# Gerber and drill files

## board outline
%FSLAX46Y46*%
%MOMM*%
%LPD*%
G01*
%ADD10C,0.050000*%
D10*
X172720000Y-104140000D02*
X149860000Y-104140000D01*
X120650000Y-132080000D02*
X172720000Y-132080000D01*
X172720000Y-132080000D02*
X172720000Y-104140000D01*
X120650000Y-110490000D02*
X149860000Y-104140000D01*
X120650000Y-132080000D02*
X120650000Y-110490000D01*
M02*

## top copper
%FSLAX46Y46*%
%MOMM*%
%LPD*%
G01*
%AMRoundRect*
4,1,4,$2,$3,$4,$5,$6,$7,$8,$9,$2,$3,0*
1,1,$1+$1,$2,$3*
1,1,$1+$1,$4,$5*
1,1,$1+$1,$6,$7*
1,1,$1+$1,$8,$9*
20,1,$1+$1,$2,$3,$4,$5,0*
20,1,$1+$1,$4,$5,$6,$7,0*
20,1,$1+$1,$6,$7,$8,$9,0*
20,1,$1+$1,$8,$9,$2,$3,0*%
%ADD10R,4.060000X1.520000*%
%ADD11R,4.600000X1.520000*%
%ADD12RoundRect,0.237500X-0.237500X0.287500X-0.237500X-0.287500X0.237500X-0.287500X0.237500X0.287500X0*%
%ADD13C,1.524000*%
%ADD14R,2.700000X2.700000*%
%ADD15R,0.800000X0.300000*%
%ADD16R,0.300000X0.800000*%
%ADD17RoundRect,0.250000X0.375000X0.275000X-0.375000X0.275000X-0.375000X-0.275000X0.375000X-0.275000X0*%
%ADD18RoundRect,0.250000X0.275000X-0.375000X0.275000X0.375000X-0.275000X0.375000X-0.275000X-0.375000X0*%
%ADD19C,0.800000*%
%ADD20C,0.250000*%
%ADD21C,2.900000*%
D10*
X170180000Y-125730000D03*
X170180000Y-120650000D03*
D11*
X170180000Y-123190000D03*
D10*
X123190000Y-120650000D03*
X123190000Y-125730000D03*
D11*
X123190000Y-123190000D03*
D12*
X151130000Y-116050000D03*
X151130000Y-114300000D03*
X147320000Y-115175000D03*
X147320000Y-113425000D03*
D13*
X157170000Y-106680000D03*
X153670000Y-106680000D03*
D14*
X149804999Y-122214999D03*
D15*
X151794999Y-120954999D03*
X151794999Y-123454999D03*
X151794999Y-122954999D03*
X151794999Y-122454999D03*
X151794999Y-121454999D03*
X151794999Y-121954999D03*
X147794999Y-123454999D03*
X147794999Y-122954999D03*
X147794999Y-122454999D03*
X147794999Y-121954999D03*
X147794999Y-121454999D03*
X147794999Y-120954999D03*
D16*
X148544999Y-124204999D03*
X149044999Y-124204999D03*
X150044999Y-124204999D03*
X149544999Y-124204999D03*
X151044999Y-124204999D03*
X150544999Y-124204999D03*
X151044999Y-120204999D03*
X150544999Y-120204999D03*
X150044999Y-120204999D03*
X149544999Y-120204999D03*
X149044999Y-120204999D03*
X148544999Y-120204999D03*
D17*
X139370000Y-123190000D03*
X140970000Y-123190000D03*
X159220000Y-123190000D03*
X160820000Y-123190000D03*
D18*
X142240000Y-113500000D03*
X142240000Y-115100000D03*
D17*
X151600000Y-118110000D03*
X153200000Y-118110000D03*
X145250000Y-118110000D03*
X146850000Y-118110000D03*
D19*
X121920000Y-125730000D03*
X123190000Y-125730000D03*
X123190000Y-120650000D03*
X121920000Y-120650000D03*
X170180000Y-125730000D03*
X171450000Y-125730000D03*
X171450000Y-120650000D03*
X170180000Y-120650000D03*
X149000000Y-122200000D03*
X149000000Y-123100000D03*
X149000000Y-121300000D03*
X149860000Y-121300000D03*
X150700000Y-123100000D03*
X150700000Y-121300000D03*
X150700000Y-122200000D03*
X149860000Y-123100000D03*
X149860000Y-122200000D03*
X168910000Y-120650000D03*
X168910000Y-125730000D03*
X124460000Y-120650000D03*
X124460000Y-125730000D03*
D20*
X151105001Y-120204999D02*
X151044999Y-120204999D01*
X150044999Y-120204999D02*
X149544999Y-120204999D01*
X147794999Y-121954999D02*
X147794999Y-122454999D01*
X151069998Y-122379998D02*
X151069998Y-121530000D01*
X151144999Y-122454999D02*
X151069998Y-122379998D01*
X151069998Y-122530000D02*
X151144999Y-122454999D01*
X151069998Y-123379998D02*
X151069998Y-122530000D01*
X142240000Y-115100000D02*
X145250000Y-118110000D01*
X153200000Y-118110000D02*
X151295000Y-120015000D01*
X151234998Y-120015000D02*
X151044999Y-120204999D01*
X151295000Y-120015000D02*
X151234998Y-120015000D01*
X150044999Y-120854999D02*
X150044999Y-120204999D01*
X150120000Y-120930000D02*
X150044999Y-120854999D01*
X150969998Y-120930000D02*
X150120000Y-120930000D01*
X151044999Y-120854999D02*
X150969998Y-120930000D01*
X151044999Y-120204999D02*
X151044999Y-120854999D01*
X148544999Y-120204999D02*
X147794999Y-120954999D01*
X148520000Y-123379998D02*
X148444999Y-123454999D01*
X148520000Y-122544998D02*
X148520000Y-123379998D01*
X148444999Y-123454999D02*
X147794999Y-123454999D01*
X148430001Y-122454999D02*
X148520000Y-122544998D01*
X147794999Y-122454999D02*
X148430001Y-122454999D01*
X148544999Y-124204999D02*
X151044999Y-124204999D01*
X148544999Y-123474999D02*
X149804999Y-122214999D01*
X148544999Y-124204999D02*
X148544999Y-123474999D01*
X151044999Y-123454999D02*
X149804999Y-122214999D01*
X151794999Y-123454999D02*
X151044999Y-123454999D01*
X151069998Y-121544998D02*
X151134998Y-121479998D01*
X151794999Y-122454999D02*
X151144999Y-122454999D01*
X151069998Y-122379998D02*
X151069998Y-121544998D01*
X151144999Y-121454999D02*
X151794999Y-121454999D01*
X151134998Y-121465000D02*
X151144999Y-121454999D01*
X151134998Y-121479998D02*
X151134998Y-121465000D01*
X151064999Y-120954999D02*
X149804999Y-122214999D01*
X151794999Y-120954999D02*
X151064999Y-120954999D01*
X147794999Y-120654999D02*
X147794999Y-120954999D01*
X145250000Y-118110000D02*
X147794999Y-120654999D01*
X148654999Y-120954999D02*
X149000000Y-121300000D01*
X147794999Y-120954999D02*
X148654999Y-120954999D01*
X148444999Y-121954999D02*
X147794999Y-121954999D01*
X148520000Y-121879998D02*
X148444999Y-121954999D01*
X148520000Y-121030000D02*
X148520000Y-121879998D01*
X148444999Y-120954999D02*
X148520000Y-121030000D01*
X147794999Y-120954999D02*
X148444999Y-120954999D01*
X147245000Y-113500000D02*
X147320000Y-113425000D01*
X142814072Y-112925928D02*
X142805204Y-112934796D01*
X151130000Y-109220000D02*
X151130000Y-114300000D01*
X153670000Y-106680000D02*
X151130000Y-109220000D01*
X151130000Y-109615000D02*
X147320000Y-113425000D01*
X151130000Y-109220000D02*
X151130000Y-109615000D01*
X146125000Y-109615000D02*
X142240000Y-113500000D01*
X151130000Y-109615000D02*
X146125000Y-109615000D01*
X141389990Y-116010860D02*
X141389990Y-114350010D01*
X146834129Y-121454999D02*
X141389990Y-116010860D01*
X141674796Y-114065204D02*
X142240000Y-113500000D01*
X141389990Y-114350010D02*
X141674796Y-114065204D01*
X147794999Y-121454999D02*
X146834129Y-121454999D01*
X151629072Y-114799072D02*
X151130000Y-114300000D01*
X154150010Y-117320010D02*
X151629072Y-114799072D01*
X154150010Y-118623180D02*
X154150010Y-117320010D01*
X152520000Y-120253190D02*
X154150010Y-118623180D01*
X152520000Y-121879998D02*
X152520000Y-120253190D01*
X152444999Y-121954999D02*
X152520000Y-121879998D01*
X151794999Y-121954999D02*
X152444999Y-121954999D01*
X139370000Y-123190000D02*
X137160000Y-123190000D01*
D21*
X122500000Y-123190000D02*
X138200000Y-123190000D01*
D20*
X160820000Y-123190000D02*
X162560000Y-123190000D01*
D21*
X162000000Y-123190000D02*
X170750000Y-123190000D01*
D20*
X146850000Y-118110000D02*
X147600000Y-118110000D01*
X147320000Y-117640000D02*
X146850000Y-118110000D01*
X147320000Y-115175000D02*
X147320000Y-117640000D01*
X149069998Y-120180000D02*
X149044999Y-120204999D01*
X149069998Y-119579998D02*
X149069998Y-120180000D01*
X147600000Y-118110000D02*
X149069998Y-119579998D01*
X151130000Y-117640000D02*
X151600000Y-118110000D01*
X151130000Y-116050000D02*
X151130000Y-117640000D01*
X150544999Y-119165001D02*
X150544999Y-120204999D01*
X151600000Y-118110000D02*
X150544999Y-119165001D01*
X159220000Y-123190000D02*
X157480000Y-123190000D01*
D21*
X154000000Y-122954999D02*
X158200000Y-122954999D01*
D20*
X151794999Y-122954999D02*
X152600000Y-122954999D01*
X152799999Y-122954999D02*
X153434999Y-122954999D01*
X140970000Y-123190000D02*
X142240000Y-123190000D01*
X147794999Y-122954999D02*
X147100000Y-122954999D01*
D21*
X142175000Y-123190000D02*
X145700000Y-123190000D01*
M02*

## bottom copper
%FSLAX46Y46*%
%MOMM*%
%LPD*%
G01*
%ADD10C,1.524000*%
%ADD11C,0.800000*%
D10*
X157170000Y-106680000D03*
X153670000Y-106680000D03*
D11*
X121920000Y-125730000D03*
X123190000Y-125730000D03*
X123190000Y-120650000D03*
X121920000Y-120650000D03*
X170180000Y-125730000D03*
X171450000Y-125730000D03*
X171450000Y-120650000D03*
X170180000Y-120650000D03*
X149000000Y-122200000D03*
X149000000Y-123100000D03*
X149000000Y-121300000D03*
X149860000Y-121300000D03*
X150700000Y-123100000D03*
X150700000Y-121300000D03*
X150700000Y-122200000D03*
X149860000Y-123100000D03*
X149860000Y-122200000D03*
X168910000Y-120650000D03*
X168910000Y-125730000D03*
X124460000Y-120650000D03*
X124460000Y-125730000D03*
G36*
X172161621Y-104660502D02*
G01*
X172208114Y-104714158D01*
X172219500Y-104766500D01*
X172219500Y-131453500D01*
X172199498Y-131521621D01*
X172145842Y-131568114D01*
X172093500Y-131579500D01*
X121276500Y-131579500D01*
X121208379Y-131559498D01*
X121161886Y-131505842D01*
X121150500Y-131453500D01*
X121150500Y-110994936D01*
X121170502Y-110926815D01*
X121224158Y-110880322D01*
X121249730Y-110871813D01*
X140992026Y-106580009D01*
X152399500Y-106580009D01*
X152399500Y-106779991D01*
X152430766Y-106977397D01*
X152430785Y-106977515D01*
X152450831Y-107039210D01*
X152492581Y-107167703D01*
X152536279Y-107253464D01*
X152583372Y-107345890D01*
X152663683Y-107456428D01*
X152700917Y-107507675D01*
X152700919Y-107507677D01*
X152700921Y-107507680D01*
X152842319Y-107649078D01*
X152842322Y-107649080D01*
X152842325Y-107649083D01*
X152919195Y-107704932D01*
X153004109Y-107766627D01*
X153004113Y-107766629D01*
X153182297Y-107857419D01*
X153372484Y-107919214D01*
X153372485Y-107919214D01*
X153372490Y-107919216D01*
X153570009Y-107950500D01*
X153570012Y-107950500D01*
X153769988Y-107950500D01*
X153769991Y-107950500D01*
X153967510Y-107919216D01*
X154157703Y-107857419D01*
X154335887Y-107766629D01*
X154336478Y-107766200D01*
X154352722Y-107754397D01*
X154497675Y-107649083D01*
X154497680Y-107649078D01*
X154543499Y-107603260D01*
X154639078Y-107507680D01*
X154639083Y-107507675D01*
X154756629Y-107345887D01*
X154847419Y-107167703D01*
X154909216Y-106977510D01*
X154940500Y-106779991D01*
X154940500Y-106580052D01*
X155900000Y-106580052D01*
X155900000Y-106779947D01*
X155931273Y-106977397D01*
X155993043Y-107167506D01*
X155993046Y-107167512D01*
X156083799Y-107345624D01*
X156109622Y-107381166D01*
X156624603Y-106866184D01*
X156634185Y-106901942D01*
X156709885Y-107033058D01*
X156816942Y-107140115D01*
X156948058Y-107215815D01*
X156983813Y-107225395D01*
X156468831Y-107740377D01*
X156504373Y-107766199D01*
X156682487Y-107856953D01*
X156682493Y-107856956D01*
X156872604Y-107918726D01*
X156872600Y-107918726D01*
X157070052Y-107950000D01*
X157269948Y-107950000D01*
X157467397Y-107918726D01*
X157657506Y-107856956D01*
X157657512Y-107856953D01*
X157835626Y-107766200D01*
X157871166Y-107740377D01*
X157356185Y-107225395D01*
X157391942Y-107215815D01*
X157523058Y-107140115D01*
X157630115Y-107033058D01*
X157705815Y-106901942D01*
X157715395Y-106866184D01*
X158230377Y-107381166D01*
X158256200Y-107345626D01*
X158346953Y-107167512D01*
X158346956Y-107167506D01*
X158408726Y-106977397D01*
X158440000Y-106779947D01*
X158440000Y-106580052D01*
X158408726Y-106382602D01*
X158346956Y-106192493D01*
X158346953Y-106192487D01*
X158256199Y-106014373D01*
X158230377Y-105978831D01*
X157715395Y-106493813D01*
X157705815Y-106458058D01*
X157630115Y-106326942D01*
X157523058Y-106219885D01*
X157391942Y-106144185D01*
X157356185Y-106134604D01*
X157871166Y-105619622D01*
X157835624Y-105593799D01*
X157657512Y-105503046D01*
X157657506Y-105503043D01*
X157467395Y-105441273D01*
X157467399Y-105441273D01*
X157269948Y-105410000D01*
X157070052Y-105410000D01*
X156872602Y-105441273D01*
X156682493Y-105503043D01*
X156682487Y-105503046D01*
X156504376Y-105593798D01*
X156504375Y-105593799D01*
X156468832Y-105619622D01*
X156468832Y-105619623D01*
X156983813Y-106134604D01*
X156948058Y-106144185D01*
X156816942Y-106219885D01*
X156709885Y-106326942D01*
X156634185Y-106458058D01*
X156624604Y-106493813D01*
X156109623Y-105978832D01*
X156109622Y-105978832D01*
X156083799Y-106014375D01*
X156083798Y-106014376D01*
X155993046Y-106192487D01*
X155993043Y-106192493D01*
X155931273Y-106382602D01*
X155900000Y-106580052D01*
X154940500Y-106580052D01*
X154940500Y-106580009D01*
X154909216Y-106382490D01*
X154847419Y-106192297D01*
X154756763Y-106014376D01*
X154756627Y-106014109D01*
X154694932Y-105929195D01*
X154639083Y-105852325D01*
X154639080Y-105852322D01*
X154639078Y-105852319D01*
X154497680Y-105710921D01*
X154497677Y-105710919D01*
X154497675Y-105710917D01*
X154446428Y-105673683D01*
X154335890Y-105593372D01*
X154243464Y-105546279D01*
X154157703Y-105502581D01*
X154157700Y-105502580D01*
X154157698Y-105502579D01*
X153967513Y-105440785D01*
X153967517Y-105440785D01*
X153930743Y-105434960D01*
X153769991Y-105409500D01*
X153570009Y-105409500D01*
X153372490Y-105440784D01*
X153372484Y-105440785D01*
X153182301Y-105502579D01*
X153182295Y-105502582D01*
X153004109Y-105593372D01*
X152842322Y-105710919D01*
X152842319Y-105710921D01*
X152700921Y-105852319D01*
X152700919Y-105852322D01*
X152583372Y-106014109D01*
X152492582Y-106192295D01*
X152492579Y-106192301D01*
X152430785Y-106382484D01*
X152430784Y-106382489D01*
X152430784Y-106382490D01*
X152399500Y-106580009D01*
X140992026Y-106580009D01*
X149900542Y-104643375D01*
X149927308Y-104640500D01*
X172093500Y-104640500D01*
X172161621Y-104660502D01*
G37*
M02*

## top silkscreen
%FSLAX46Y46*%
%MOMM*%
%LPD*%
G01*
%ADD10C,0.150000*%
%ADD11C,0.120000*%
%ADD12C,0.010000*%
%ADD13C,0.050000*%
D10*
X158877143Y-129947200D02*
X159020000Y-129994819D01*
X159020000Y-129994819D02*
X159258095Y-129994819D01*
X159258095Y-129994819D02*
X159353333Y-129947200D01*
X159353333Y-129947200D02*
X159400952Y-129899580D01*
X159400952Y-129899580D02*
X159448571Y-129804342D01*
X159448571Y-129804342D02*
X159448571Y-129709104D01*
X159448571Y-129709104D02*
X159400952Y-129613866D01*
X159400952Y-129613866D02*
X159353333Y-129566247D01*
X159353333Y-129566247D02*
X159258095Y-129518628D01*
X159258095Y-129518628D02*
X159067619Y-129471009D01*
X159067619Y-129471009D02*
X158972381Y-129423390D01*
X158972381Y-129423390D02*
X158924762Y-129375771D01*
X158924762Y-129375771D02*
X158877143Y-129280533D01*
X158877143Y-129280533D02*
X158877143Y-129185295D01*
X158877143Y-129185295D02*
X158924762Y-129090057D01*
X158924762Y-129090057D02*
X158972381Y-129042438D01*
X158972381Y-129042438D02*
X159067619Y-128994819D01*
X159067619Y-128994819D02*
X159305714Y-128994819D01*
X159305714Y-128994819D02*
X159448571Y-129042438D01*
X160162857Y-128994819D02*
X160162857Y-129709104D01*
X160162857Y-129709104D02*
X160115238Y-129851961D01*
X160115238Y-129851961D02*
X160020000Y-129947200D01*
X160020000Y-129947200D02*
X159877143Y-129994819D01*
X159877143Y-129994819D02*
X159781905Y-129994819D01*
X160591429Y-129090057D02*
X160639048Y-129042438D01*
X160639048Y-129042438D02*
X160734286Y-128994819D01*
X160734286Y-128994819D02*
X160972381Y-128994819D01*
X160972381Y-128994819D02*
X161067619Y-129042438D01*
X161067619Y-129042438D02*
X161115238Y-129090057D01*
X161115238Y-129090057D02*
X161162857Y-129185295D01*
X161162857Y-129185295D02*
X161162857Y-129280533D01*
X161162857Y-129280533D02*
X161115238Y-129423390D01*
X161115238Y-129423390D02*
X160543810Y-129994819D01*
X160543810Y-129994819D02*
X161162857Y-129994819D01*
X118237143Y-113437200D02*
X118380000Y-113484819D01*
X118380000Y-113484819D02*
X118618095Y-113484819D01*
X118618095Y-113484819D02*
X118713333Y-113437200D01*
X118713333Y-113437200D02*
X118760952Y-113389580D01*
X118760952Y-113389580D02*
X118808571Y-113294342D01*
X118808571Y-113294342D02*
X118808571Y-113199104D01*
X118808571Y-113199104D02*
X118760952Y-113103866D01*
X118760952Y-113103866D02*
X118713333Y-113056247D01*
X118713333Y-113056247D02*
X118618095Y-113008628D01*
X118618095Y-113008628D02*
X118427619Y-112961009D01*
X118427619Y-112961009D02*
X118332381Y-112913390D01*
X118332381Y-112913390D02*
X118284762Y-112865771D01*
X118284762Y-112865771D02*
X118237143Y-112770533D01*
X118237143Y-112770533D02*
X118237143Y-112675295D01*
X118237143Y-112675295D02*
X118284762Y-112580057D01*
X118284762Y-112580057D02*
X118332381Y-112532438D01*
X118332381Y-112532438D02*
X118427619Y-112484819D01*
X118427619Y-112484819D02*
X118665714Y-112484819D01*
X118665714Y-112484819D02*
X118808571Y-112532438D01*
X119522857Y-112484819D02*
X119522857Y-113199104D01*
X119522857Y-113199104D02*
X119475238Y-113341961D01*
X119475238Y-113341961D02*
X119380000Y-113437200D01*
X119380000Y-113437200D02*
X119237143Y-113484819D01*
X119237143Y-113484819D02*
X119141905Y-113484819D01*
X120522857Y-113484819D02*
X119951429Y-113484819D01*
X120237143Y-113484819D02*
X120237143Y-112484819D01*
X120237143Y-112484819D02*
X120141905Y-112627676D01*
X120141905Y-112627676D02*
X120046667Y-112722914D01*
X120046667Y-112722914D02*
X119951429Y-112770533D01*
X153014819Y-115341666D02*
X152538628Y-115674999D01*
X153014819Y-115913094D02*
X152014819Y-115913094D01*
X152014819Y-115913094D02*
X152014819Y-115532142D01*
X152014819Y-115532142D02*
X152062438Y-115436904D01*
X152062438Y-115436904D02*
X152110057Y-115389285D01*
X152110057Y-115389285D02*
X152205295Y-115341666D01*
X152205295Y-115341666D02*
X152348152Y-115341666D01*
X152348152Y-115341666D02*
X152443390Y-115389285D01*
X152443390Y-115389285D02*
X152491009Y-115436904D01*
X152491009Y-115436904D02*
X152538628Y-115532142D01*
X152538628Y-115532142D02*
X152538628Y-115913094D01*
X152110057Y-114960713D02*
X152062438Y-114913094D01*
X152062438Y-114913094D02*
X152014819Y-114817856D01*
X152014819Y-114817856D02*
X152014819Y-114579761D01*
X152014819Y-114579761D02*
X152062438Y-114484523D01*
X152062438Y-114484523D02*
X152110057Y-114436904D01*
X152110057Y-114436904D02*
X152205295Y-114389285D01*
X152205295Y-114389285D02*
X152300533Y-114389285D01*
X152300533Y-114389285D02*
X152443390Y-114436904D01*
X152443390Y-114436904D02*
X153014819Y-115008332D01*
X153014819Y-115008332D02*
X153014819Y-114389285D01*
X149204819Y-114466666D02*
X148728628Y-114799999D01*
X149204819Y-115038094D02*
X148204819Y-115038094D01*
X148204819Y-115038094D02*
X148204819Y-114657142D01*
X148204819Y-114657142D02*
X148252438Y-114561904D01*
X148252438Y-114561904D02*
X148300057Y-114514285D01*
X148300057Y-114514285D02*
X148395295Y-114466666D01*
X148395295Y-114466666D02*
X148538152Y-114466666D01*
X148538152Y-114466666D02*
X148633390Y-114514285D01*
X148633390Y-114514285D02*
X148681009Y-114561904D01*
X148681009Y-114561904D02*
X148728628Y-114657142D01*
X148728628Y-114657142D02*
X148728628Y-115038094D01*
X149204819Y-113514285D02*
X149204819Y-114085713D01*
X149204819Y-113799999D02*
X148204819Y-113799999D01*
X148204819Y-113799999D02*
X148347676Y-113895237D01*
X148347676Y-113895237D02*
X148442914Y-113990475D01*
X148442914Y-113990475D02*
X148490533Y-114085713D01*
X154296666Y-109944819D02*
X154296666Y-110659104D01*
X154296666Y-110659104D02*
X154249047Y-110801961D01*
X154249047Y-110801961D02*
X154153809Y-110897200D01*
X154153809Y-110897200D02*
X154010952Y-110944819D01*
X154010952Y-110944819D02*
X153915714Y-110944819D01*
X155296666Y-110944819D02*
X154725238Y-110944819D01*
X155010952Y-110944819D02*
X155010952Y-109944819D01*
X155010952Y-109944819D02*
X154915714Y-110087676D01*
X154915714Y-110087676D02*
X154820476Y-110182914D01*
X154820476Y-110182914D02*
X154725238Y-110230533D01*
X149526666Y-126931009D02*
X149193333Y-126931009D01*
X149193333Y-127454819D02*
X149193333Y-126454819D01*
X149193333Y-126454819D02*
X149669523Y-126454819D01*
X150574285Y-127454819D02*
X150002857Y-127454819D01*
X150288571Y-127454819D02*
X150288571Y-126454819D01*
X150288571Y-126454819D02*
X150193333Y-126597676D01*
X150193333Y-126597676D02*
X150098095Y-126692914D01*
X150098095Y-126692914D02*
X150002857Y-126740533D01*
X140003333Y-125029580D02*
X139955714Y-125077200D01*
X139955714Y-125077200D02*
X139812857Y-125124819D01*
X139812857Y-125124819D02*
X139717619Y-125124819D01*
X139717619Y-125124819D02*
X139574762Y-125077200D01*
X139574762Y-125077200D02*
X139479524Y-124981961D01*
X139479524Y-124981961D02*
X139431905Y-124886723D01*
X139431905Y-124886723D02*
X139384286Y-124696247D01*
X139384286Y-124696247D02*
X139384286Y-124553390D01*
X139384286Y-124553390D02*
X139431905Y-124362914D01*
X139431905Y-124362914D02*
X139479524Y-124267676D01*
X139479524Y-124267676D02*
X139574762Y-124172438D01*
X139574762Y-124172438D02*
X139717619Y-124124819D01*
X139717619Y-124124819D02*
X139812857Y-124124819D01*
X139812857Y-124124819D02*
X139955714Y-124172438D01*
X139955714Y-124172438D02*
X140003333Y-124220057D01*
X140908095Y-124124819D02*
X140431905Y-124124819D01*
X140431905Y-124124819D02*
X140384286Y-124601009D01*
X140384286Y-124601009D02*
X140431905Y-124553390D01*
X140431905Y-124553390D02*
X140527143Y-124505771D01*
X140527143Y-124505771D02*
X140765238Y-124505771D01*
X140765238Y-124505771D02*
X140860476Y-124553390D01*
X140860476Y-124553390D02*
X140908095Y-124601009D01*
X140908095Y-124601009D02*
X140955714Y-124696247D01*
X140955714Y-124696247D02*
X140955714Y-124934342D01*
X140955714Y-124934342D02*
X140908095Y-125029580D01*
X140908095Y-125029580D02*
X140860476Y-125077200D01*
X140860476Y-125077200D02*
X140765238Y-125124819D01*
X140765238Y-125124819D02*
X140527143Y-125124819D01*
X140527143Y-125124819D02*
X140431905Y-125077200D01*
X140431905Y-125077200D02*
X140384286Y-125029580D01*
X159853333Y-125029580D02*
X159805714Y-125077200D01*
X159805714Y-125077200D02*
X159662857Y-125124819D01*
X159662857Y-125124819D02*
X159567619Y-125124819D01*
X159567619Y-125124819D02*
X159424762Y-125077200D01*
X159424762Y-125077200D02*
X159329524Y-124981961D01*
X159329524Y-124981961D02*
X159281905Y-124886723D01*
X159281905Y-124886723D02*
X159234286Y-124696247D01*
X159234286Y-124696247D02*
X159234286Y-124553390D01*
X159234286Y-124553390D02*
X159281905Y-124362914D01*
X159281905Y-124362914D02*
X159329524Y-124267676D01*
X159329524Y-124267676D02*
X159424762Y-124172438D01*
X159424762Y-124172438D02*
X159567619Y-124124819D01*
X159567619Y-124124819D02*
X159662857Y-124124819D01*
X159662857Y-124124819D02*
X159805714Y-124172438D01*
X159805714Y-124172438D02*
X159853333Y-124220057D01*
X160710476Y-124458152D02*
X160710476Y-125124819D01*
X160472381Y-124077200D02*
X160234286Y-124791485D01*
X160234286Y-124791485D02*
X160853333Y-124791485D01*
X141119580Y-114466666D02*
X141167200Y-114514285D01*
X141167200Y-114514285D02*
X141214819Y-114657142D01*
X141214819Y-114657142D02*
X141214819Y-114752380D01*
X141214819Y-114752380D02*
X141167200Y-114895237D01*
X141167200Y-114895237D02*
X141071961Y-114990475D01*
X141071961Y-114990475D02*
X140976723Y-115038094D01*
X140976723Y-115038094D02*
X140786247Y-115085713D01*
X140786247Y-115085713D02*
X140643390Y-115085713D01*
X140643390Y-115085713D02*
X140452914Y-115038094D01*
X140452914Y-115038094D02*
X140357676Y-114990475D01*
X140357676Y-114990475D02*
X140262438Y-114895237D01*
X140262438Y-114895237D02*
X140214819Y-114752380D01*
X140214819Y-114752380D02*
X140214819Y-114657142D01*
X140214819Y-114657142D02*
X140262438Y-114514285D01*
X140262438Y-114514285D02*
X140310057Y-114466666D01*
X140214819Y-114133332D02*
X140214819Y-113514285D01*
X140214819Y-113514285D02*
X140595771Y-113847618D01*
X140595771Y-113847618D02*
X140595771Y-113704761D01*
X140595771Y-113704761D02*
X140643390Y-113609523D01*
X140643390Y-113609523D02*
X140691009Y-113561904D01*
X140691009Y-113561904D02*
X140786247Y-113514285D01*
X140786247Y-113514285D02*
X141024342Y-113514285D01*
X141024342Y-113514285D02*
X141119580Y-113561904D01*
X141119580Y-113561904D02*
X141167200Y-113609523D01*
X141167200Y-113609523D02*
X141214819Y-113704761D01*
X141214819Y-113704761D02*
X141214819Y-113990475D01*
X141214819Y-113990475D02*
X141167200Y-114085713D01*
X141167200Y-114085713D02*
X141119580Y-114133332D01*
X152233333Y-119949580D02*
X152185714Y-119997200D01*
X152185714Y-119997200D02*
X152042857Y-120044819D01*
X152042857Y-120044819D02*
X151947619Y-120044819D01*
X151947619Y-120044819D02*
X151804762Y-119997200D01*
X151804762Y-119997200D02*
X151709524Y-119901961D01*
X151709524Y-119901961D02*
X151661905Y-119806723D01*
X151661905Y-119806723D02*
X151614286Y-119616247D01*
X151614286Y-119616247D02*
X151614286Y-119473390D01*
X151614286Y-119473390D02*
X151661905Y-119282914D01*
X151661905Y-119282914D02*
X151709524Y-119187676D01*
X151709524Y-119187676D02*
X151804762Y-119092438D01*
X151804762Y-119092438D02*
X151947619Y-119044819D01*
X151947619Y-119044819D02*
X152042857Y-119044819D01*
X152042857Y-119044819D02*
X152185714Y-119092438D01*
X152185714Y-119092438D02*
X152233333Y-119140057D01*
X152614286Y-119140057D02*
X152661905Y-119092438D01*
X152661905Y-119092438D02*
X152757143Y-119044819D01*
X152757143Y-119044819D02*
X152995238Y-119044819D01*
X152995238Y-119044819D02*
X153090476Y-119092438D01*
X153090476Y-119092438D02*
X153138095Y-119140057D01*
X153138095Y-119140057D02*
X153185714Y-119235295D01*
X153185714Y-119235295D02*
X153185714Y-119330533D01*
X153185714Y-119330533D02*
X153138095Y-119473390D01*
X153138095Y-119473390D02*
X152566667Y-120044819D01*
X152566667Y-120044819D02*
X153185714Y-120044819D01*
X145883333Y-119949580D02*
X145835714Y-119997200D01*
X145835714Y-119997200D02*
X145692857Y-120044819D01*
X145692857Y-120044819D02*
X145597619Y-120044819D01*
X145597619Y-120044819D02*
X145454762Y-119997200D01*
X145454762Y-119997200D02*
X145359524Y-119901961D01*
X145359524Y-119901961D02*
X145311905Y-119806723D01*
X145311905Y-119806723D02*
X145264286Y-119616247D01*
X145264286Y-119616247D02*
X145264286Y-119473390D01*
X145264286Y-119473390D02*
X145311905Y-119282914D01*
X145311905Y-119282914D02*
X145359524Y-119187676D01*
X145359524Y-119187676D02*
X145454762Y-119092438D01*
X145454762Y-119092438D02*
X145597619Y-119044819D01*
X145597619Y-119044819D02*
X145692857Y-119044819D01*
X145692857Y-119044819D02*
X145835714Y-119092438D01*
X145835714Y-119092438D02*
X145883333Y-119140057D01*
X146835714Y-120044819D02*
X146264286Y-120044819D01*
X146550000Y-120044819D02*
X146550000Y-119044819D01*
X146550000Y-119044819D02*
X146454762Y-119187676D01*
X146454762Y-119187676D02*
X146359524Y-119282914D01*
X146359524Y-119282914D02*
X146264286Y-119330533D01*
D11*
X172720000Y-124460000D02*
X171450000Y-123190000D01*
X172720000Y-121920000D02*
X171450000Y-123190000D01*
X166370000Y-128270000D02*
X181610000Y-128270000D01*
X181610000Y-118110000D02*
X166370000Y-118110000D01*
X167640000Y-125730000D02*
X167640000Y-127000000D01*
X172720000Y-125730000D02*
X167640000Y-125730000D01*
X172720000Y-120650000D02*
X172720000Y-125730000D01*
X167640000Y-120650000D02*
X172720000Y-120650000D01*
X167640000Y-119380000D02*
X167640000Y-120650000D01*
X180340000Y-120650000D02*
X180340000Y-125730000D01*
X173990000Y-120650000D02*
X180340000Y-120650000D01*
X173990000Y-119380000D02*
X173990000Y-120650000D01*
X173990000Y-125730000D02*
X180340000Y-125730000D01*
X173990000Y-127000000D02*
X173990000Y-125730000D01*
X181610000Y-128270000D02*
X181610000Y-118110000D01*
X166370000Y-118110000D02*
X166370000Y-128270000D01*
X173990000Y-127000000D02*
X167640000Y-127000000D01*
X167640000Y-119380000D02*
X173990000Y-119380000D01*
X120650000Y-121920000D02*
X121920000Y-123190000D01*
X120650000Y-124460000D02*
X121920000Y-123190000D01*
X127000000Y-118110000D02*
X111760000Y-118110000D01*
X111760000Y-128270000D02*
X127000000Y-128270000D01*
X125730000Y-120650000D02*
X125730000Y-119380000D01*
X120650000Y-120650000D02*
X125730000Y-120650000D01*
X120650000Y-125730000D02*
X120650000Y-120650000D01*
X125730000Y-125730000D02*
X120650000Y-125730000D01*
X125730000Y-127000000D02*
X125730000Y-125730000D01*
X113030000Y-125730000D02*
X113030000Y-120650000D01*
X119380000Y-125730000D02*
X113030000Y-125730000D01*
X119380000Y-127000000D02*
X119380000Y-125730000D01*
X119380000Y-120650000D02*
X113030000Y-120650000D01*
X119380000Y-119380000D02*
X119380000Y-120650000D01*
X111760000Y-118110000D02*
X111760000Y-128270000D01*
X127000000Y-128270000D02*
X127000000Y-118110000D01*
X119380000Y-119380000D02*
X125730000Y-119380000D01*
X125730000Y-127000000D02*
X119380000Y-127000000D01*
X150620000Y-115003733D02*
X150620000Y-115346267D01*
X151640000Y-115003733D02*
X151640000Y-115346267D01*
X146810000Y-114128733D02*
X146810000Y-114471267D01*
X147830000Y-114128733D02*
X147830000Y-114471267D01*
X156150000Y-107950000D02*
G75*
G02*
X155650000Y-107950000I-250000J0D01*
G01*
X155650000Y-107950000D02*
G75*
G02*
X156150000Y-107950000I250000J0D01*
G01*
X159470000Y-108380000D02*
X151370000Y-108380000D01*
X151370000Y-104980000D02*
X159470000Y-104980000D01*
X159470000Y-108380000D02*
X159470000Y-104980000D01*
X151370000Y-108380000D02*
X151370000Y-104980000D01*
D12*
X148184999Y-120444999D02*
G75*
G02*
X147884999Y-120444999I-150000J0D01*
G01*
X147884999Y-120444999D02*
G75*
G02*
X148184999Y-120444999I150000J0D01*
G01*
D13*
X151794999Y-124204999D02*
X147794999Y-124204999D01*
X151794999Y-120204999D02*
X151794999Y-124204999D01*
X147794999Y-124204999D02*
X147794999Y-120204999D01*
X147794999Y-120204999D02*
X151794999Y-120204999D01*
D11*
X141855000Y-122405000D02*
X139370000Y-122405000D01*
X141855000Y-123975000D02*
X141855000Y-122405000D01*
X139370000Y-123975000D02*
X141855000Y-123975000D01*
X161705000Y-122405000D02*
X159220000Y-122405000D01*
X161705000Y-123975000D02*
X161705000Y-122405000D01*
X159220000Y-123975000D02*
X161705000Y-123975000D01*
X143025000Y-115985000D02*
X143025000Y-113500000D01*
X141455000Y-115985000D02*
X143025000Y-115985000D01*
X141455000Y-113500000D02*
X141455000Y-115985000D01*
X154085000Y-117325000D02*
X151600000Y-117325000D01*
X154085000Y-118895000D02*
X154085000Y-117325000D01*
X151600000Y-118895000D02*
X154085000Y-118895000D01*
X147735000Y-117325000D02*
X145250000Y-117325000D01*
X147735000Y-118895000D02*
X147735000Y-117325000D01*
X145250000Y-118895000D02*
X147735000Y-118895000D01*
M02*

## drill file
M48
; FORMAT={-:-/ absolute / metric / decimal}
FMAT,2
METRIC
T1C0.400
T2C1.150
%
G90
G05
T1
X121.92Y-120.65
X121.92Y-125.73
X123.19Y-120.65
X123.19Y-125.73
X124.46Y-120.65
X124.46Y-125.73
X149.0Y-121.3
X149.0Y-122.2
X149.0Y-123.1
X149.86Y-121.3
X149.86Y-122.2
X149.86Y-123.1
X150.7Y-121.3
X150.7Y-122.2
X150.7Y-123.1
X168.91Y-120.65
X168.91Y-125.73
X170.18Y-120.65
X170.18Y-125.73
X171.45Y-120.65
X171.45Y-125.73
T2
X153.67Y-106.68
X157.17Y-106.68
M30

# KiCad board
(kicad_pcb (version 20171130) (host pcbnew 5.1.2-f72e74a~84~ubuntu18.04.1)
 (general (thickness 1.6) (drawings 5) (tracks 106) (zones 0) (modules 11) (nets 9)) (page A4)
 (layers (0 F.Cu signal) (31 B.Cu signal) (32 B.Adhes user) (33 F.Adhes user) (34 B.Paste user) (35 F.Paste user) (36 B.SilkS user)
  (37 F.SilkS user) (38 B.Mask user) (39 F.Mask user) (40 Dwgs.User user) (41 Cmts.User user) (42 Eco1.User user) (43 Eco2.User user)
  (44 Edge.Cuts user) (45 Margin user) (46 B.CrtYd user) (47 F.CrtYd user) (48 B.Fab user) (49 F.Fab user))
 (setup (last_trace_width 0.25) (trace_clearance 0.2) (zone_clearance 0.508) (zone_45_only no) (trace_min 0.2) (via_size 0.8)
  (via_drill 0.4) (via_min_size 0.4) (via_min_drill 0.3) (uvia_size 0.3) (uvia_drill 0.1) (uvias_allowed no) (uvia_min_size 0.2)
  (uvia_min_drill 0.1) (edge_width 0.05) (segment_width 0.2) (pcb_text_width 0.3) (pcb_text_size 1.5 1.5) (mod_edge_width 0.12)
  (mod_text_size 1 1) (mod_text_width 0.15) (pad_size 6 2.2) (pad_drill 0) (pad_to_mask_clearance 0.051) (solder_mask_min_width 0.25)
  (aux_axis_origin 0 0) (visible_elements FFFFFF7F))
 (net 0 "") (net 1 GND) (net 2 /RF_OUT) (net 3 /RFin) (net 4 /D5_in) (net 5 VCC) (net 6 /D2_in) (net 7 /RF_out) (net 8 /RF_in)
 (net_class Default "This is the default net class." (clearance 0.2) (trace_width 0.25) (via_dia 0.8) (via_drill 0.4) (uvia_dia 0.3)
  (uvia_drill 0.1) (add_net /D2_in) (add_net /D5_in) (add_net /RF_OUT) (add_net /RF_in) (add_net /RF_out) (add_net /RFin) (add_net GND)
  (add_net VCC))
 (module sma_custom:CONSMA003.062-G (layer F.Cu) (at 173.99 125.73)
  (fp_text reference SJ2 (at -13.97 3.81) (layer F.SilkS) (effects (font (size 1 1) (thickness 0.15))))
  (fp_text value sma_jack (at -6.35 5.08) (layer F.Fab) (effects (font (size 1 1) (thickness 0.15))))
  (fp_line (start -1.27 -1.27) (end -2.54 -2.54) (layer F.SilkS) (width 0.12))
  (fp_line (start -1.27 -3.81) (end -2.54 -2.54) (layer F.SilkS) (width 0.12))
  (fp_line (start -7.62 2.54) (end 7.62 2.54) (layer F.SilkS) (width 0.12))
  (fp_line (start 7.62 -7.62) (end -7.62 -7.62) (layer F.SilkS) (width 0.12))
  (fp_line (start -6.35 0) (end -6.35 1.27) (layer F.SilkS) (width 0.12))
  (fp_line (start -1.27 0) (end -6.35 0) (layer F.SilkS) (width 0.12))
  (fp_line (start -1.27 -5.08) (end -1.27 0) (layer F.SilkS) (width 0.12))
  (fp_line (start -6.35 -5.08) (end -1.27 -5.08) (layer F.SilkS) (width 0.12))
  (fp_line (start -6.35 -6.35) (end -6.35 -5.08) (layer F.SilkS) (width 0.12))
  (fp_line (start 6.35 -5.08) (end 6.35 0) (layer F.SilkS) (width 0.12))
  (fp_line (start 0 -5.08) (end 6.35 -5.08) (layer F.SilkS) (width 0.12))
  (fp_line (start 0 -6.35) (end 0 -5.08) (layer F.SilkS) (width 0.12))
  (fp_line (start 0 0) (end 6.35 0) (layer F.SilkS) (width 0.12))
  (fp_line (start 0 1.27) (end 0 0) (layer F.SilkS) (width 0.12))
  (fp_line (start 7.62 2.54) (end 7.62 -7.62) (layer F.SilkS) (width 0.12))
  (fp_line (start -7.62 -7.62) (end -7.62 2.54) (layer F.SilkS) (width 0.12))
  (fp_line (start 0 1.27) (end -6.35 1.27) (layer F.SilkS) (width 0.12))
  (fp_line (start -6.35 -6.35) (end 0 -6.35) (layer F.SilkS) (width 0.12))
  (pad 3 smd rect (at -3.81 0) (size 4.06 1.52) (layers F.Cu F.Paste F.Mask) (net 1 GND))
  (pad 2 smd rect (at -3.81 -5.08) (size 4.06 1.52) (layers F.Cu F.Paste F.Mask) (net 1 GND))
  (pad 1 smd rect (at -3.81 -2.54) (size 4.6 1.52) (layers F.Cu F.Paste F.Mask) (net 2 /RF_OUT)))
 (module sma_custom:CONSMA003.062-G (layer F.Cu) (at 119.38 120.65 180)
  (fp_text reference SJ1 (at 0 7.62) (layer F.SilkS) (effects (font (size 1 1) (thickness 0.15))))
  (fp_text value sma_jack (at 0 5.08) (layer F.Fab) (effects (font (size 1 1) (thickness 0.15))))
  (fp_line (start -1.27 -1.27) (end -2.54 -2.54) (layer F.SilkS) (width 0.12))
  (fp_line (start -1.27 -3.81) (end -2.54 -2.54) (layer F.SilkS) (width 0.12))
  (fp_line (start -7.62 2.54) (end 7.62 2.54) (layer F.SilkS) (width 0.12))
  (fp_line (start 7.62 -7.62) (end -7.62 -7.62) (layer F.SilkS) (width 0.12))
  (fp_line (start -6.35 0) (end -6.35 1.27) (layer F.SilkS) (width 0.12))
  (fp_line (start -1.27 0) (end -6.35 0) (layer F.SilkS) (width 0.12))
  (fp_line (start -1.27 -5.08) (end -1.27 0) (layer F.SilkS) (width 0.12))
  (fp_line (start -6.35 -5.08) (end -1.27 -5.08) (layer F.SilkS) (width 0.12))
  (fp_line (start -6.35 -6.35) (end -6.35 -5.08) (layer F.SilkS) (width 0.12))
  (fp_line (start 6.35 -5.08) (end 6.35 0) (layer F.SilkS) (width 0.12))
  (fp_line (start 0 -5.08) (end 6.35 -5.08) (layer F.SilkS) (width 0.12))
  (fp_line (start 0 -6.35) (end 0 -5.08) (layer F.SilkS) (width 0.12))
  (fp_line (start 0 0) (end 6.35 0) (layer F.SilkS) (width 0.12))
  (fp_line (start 0 1.27) (end 0 0) (layer F.SilkS) (width 0.12))
  (fp_line (start 7.62 2.54) (end 7.62 -7.62) (layer F.SilkS) (width 0.12))
  (fp_line (start -7.62 -7.62) (end -7.62 2.54) (layer F.SilkS) (width 0.12))
  (fp_line (start 0 1.27) (end -6.35 1.27) (layer F.SilkS) (width 0.12))
  (fp_line (start -6.35 -6.35) (end 0 -6.35) (layer F.SilkS) (width 0.12))
  (pad 3 smd rect (at -3.81 0 180) (size 4.06 1.52) (layers F.Cu F.Paste F.Mask) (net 1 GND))
  (pad 2 smd rect (at -3.81 -5.08 180) (size 4.06 1.52) (layers F.Cu F.Paste F.Mask) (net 1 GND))
  (pad 1 smd rect (at -3.81 -2.54 180) (size 4.6 1.52) (layers F.Cu F.Paste F.Mask) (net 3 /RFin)))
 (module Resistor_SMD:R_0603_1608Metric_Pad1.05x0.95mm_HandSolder (layer F.Cu) (at 151.13 115.175 270)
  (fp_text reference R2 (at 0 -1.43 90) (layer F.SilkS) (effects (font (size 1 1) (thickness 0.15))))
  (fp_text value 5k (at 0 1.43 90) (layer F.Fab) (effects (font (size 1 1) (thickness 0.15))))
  (fp_line (start -0.171267 0.51) (end 0.171267 0.51) (layer F.SilkS) (width 0.12))
  (fp_line (start -0.171267 -0.51) (end 0.171267 -0.51) (layer F.SilkS) (width 0.12))
  (pad 2 smd roundrect (at 0.875 0 270) (size 1.05 0.95) (layers F.Cu F.Paste F.Mask) (roundrect_rratio 0.25) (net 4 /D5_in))
  (pad 1 smd roundrect (at -0.875 0 270) (size 1.05 0.95) (layers F.Cu F.Paste F.Mask) (roundrect_rratio 0.25) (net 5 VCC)))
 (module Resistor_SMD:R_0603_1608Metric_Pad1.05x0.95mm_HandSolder (layer F.Cu) (at 147.32 114.3 270)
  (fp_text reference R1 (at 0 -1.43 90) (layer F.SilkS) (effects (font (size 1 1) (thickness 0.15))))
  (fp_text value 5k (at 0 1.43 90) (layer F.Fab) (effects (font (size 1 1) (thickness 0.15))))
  (fp_line (start -0.171267 0.51) (end 0.171267 0.51) (layer F.SilkS) (width 0.12))
  (fp_line (start -0.171267 -0.51) (end 0.171267 -0.51) (layer F.SilkS) (width 0.12))
  (pad 2 smd roundrect (at 0.875 0 270) (size 1.05 0.95) (layers F.Cu F.Paste F.Mask) (roundrect_rratio 0.25) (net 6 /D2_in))
  (pad 1 smd roundrect (at -0.875 0 270) (size 1.05 0.95) (layers F.Cu F.Paste F.Mask) (roundrect_rratio 0.25) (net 5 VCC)))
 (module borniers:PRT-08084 (layer F.Cu) (at 157.17 111.76)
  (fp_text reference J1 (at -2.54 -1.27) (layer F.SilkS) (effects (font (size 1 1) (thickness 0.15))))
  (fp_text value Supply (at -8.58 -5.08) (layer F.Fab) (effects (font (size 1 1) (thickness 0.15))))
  (fp_circle (center -1.27 -3.81) (end -1.02 -3.81) (layer F.SilkS) (width 0.12))
  (fp_line (start 2.3 -3.38) (end -5.8 -3.38) (layer F.SilkS) (width 0.12))
  (fp_line (start -5.8 -6.78) (end 2.3 -6.78) (layer F.SilkS) (width 0.12))
  (fp_line (start 2.3 -3.38) (end 2.3 -6.78) (layer F.SilkS) (width 0.12))
  (fp_line (start -5.8 -3.38) (end -5.8 -6.78) (layer F.SilkS) (width 0.12))
  (pad 2 thru_hole circle (at 0 -5.08) (size 1.524 1.524) (drill 1.15) (layers *.Cu *.Mask) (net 1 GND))
  (pad 1 thru_hole circle (at -3.5 -5.08) (size 1.524 1.524) (drill 1.15) (layers *.Cu *.Mask) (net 5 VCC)))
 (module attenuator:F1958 (layer F.Cu) (at 150.334999 122.744999)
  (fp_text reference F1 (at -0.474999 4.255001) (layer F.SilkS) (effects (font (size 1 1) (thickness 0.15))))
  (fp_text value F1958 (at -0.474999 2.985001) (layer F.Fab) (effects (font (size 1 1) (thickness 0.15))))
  (fp_circle (center -2.3 -2.3) (end -2.15 -2.3) (layer F.SilkS) (width 0.01))
  (fp_line (start 1.46 1.46) (end -2.54 1.46) (layer F.SilkS) (width 0.05))
  (fp_line (start 1.46 -2.54) (end 1.46 1.46) (layer F.SilkS) (width 0.05))
  (fp_line (start -2.54 1.46) (end -2.54 -2.54) (layer F.SilkS) (width 0.05))
  (fp_line (start -2.54 -2.54) (end 1.46 -2.54) (layer F.SilkS) (width 0.05))
  (pad 25 smd rect (at -0.53 -0.53) (size 2.7 2.7) (layers F.Cu F.Paste F.Mask) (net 1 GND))
  (pad 18 smd rect (at 1.46 -1.79 90) (size 0.3 0.8) (layers F.Cu F.Paste F.Mask) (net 1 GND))
  (pad 13 smd rect (at 1.46 0.71 90) (size 0.3 0.8) (layers F.Cu F.Paste F.Mask) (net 1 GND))
  (pad 14 smd rect (at 1.46 0.21 90) (size 0.3 0.8) (layers F.Cu F.Paste F.Mask) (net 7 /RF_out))
  (pad 15 smd rect (at 1.46 -0.29 90) (size 0.3 0.8) (layers F.Cu F.Paste F.Mask) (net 1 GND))
  (pad 17 smd rect (at 1.46 -1.29 90) (size 0.3 0.8) (layers F.Cu F.Paste F.Mask) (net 1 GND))
  (pad 16 smd rect (at 1.46 -0.79 90) (size 0.3 0.8) (layers F.Cu F.Paste F.Mask) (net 5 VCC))
  (pad 6 smd rect (at -2.54 0.71 90) (size 0.3 0.8) (layers F.Cu F.Paste F.Mask) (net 1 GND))
  (pad 5 smd rect (at -2.54 0.21 90) (size 0.3 0.8) (layers F.Cu F.Paste F.Mask) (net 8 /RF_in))
  (pad 4 smd rect (at -2.54 -0.29 90) (size 0.3 0.8) (layers F.Cu F.Paste F.Mask) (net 1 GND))
  (pad 3 smd rect (at -2.54 -0.79 90) (size 0.3 0.8) (layers F.Cu F.Paste F.Mask) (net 1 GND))
  (pad 2 smd rect (at -2.54 -1.29 90) (size 0.3 0.8) (layers F.Cu F.Paste F.Mask) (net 5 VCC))
  (pad 1 smd rect (at -2.54 -1.79 90) (size 0.3 0.8) (layers F.Cu F.Paste F.Mask) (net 1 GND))
  (pad 7 smd rect (at -1.79 1.46) (size 0.3 0.8) (layers F.Cu F.Paste F.Mask) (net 1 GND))
  (pad 8 smd rect (at -1.29 1.46) (size 0.3 0.8) (layers F.Cu F.Paste F.Mask) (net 1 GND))
  (pad 10 smd rect (at -0.29 1.46) (size 0.3 0.8) (layers F.Cu F.Paste F.Mask) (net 1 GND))
  (pad 9 smd rect (at -0.79 1.46) (size 0.3 0.8) (layers F.Cu F.Paste F.Mask) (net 1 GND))
  (pad 12 smd rect (at 0.71 1.46) (size 0.3 0.8) (layers F.Cu F.Paste F.Mask) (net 1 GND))
  (pad 11 smd rect (at 0.21 1.46) (size 0.3 0.8) (layers F.Cu F.Paste F.Mask) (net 1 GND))
  (pad 19 smd rect (at 0.71 -2.54) (size 0.3 0.8) (layers F.Cu F.Paste F.Mask) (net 1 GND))
  (pad 20 smd rect (at 0.21 -2.54) (size 0.3 0.8) (layers F.Cu F.Paste F.Mask) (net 4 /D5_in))
  (pad 21 smd rect (at -0.29 -2.54) (size 0.3 0.8) (layers F.Cu F.Paste F.Mask) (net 1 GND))
  (pad 22 smd rect (at -0.79 -2.54) (size 0.3 0.8) (layers F.Cu F.Paste F.Mask) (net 1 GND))
  (pad 23 smd rect (at -1.29 -2.54) (size 0.3 0.8) (layers F.Cu F.Paste F.Mask) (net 6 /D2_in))
  (pad 24 smd rect (at -1.79 -2.54) (size 0.3 0.8) (layers F.Cu F.Paste F.Mask) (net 1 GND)))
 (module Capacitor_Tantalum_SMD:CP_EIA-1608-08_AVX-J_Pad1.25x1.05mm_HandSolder (layer F.Cu) (at 140.17 123.19 180)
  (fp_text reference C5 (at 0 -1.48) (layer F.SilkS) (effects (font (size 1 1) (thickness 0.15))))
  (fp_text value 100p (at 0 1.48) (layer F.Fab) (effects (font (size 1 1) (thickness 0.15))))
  (fp_line (start -1.685 0.785) (end 0.8 0.785) (layer F.SilkS) (width 0.12))
  (fp_line (start -1.685 -0.785) (end -1.685 0.785) (layer F.SilkS) (width 0.12))
  (fp_line (start 0.8 -0.785) (end -1.685 -0.785) (layer F.SilkS) (width 0.12))
  (pad 2 smd roundrect (at 0.8 0 180) (size 1.25 1.05) (layers F.Cu F.Paste F.Mask) (roundrect_rratio 0.238095) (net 3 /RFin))
  (pad 1 smd roundrect (at -0.8 0 180) (size 1.25 1.05) (layers F.Cu F.Paste F.Mask) (roundrect_rratio 0.238095) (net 8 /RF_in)))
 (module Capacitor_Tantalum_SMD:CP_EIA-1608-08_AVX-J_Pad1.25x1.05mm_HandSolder (layer F.Cu) (at 160.02 123.19 180)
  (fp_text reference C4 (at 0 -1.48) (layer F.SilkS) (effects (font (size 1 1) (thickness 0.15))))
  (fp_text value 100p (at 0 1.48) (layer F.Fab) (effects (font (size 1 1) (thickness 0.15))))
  (fp_line (start -1.685 0.785) (end 0.8 0.785) (layer F.SilkS) (width 0.12))
  (fp_line (start -1.685 -0.785) (end -1.685 0.785) (layer F.SilkS) (width 0.12))
  (fp_line (start 0.8 -0.785) (end -1.685 -0.785) (layer F.SilkS) (width 0.12))
  (pad 2 smd roundrect (at 0.8 0 180) (size 1.25 1.05) (layers F.Cu F.Paste F.Mask) (roundrect_rratio 0.238095) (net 7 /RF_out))
  (pad 1 smd roundrect (at -0.8 0 180) (size 1.25 1.05) (layers F.Cu F.Paste F.Mask) (roundrect_rratio 0.238095) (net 2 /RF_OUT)))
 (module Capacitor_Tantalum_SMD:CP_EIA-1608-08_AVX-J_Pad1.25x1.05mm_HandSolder (layer F.Cu) (at 142.24 114.3 90)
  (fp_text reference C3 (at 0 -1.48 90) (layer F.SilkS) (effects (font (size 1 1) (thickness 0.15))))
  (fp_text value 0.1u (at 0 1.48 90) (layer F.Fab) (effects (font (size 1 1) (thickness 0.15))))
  (fp_line (start -1.685 0.785) (end 0.8 0.785) (layer F.SilkS) (width 0.12))
  (fp_line (start -1.685 -0.785) (end -1.685 0.785) (layer F.SilkS) (width 0.12))
  (fp_line (start 0.8 -0.785) (end -1.685 -0.785) (layer F.SilkS) (width 0.12))
  (pad 2 smd roundrect (at 0.8 0 90) (size 1.25 1.05) (layers F.Cu F.Paste F.Mask) (roundrect_rratio 0.238095) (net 5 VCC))
  (pad 1 smd roundrect (at -0.8 0 90) (size 1.25 1.05) (layers F.Cu F.Paste F.Mask) (roundrect_rratio 0.238095) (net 1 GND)))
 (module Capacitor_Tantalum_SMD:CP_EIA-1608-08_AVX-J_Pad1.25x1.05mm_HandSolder (layer F.Cu) (at 152.4 118.11 180)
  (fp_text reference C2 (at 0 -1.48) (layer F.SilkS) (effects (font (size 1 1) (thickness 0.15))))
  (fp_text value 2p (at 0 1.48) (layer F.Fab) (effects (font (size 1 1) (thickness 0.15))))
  (fp_line (start -1.685 0.785) (end 0.8 0.785) (layer F.SilkS) (width 0.12))
  (fp_line (start -1.685 -0.785) (end -1.685 0.785) (layer F.SilkS) (width 0.12))
  (fp_line (start 0.8 -0.785) (end -1.685 -0.785) (layer F.SilkS) (width 0.12))
  (pad 2 smd roundrect (at 0.8 0 180) (size 1.25 1.05) (layers F.Cu F.Paste F.Mask) (roundrect_rratio 0.238095) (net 4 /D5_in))
  (pad 1 smd roundrect (at -0.8 0 180) (size 1.25 1.05) (layers F.Cu F.Paste F.Mask) (roundrect_rratio 0.238095) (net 1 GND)))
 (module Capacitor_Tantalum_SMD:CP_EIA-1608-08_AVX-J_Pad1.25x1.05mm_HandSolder (layer F.Cu) (at 146.05 118.11 180)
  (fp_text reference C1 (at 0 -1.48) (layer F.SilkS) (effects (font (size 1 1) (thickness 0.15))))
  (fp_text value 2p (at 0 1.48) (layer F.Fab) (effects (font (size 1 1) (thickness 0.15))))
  (fp_line (start -1.685 0.785) (end 0.8 0.785) (layer F.SilkS) (width 0.12))
  (fp_line (start -1.685 -0.785) (end -1.685 0.785) (layer F.SilkS) (width 0.12))
  (fp_line (start 0.8 -0.785) (end -1.685 -0.785) (layer F.SilkS) (width 0.12))
  (pad 2 smd roundrect (at 0.8 0 180) (size 1.25 1.05) (layers F.Cu F.Paste F.Mask) (roundrect_rratio 0.238095) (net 1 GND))
  (pad 1 smd roundrect (at -0.8 0 180) (size 1.25 1.05) (layers F.Cu F.Paste F.Mask) (roundrect_rratio 0.238095) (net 6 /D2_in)))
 (gr_line (start 172.72 104.14) (end 149.86 104.14) (layer Edge.Cuts) (width 0.05))
 (gr_line (start 120.65 132.08) (end 172.72 132.08) (layer Edge.Cuts) (width 0.05))
 (gr_line (start 172.72 132.08) (end 172.72 104.14) (layer Edge.Cuts) (width 0.05))
 (gr_line (start 120.65 110.49) (end 149.86 104.14) (layer Edge.Cuts) (width 0.05))
 (gr_line (start 120.65 132.08) (end 120.65 110.49) (layer Edge.Cuts) (width 0.05))
 (via (at 121.92 125.73) (size 0.8) (drill 0.4) (layers F.Cu B.Cu) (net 1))
 (via (at 123.19 125.73) (size 0.8) (drill 0.4) (layers F.Cu B.Cu) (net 1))
 (via (at 123.19 120.65) (size 0.8) (drill 0.4) (layers F.Cu B.Cu) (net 1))
 (via (at 121.92 120.65) (size 0.8) (drill 0.4) (layers F.Cu B.Cu) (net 1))
 (via (at 170.18 125.73) (size 0.8) (drill 0.4) (layers F.Cu B.Cu) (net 1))
 (via (at 171.45 125.73) (size 0.8) (drill 0.4) (layers F.Cu B.Cu) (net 1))
 (via (at 171.45 120.65) (size 0.8) (drill 0.4) (layers F.Cu B.Cu) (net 1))
 (via (at 170.18 120.65) (size 0.8) (drill 0.4) (layers F.Cu B.Cu) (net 1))
 (via (at 149 122.2) (size 0.8) (drill 0.4) (layers F.Cu B.Cu) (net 1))
 (via (at 149 123.1) (size 0.8) (drill 0.4) (layers F.Cu B.Cu) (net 1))
 (via (at 149 121.3) (size 0.8) (drill 0.4) (layers F.Cu B.Cu) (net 1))
 (via (at 149.86 121.3) (size 0.8) (drill 0.4) (layers F.Cu B.Cu) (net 1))
 (via (at 150.7 123.1) (size 0.8) (drill 0.4) (layers F.Cu B.Cu) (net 1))
 (via (at 150.7 121.3) (size 0.8) (drill 0.4) (layers F.Cu B.Cu) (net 1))
 (via (at 150.7 122.2) (size 0.8) (drill 0.4) (layers F.Cu B.Cu) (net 1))
 (via (at 149.86 123.1) (size 0.8) (drill 0.4) (layers F.Cu B.Cu) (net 1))
 (via (at 149.86 122.2) (size 0.8) (drill 0.4) (layers F.Cu B.Cu) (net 1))
 (segment (start 151.105001 120.204999) (end 151.044999 120.204999) (width 0.25) (layer F.Cu) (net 1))
 (segment (start 150.044999 120.204999) (end 149.544999 120.204999) (width 0.25) (layer F.Cu) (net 1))
 (segment (start 147.794999 121.954999) (end 147.794999 122.454999) (width 0.25) (layer F.Cu) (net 1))
 (segment (start 151.069998 122.379998) (end 151.069998 121.53) (width 0.25) (layer F.Cu) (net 1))
 (segment (start 151.144999 122.454999) (end 151.069998 122.379998) (width 0.25) (layer F.Cu) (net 1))
 (via (at 168.91 120.65) (size 0.8) (drill 0.4) (layers F.Cu B.Cu) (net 1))
 (via (at 168.91 125.73) (size 0.8) (drill 0.4) (layers F.Cu B.Cu) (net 1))
 (via (at 124.46 120.65) (size 0.8) (drill 0.4) (layers F.Cu B.Cu) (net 1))
 (via (at 124.46 125.73) (size 0.8) (drill 0.4) (layers F.Cu B.Cu) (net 1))
 (segment (start 151.069998 122.53) (end 151.144999 122.454999) (width 0.25) (layer F.Cu) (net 1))
 (segment (start 151.069998 123.379998) (end 151.069998 122.53) (width 0.25) (layer F.Cu) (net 1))
 (segment (start 142.24 115.1) (end 145.25 118.11) (width 0.25) (layer F.Cu) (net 1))
 (segment (start 153.2 118.11) (end 151.295 120.015) (width 0.25) (layer F.Cu) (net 1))
 (segment (start 151.234998 120.015) (end 151.044999 120.204999) (width 0.25) (layer F.Cu) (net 1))
 (segment (start 151.295 120.015) (end 151.234998 120.015) (width 0.25) (layer F.Cu) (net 1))
 (segment (start 150.044999 120.854999) (end 150.044999 120.204999) (width 0.25) (layer F.Cu) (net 1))
 (segment (start 150.12 120.93) (end 150.044999 120.854999) (width 0.25) (layer F.Cu) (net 1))
 (segment (start 150.969998 120.93) (end 150.12 120.93) (width 0.25) (layer F.Cu) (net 1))
 (segment (start 151.044999 120.854999) (end 150.969998 120.93) (width 0.25) (layer F.Cu) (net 1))
 (segment (start 151.044999 120.204999) (end 151.044999 120.854999) (width 0.25) (layer F.Cu) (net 1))
 (segment (start 148.544999 120.204999) (end 147.794999 120.954999) (width 0.25) (layer F.Cu) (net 1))
 (segment (start 148.52 123.379998) (end 148.444999 123.454999) (width 0.25) (layer F.Cu) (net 1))
 (segment (start 148.52 122.544998) (end 148.52 123.379998) (width 0.25) (layer F.Cu) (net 1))
 (segment (start 148.444999 123.454999) (end 147.794999 123.454999) (width 0.25) (layer F.Cu) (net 1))
 (segment (start 148.430001 122.454999) (end 148.52 122.544998) (width 0.25) (layer F.Cu) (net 1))
 (segment (start 147.794999 122.454999) (end 148.430001 122.454999) (width 0.25) (layer F.Cu) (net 1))
 (segment (start 148.544999 124.204999) (end 151.044999 124.204999) (width 0.25) (layer F.Cu) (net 1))
 (segment (start 148.544999 123.474999) (end 149.804999 122.214999) (width 0.25) (layer F.Cu) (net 1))
 (segment (start 148.544999 124.204999) (end 148.544999 123.474999) (width 0.25) (layer F.Cu) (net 1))
 (segment (start 151.044999 123.454999) (end 149.804999 122.214999) (width 0.25) (layer F.Cu) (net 1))
 (segment (start 151.794999 123.454999) (end 151.044999 123.454999) (width 0.25) (layer F.Cu) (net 1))
 (segment (start 151.069998 121.544998) (end 151.134998 121.479998) (width 0.25) (layer F.Cu) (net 1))
 (segment (start 151.794999 122.454999) (end 151.144999 122.454999) (width 0.25) (layer F.Cu) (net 1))
 (segment (start 151.069998 122.379998) (end 151.069998 121.544998) (width 0.25) (layer F.Cu) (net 1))
 (segment (start 151.144999 121.454999) (end 151.794999 121.454999) (width 0.25) (layer F.Cu) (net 1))
 (segment (start 151.134998 121.465) (end 151.144999 121.454999) (width 0.25) (layer F.Cu) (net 1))
 (segment (start 151.134998 121.479998) (end 151.134998 121.465) (width 0.25) (layer F.Cu) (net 1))
 (segment (start 151.064999 120.954999) (end 149.804999 122.214999) (width 0.25) (layer F.Cu) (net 1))
 (segment (start 151.794999 120.954999) (end 151.064999 120.954999) (width 0.25) (layer F.Cu) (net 1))
 (segment (start 147.794999 120.654999) (end 147.794999 120.954999) (width 0.25) (layer F.Cu) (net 1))
 (segment (start 145.25 118.11) (end 147.794999 120.654999) (width 0.25) (layer F.Cu) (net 1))
 (segment (start 148.654999 120.954999) (end 149 121.3) (width 0.25) (layer F.Cu) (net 1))
 (segment (start 147.794999 120.954999) (end 148.654999 120.954999) (width 0.25) (layer F.Cu) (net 1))
 (segment (start 148.444999 121.954999) (end 147.794999 121.954999) (width 0.25) (layer F.Cu) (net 1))
 (segment (start 148.52 121.879998) (end 148.444999 121.954999) (width 0.25) (layer F.Cu) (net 1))
 (segment (start 148.52 121.03) (end 148.52 121.879998) (width 0.25) (layer F.Cu) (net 1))
 (segment (start 148.444999 120.954999) (end 148.52 121.03) (width 0.25) (layer F.Cu) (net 1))
 (segment (start 147.794999 120.954999) (end 148.444999 120.954999) (width 0.25) (layer F.Cu) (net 1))
 (segment (start 147.245 113.5) (end 147.32 113.425) (width 0.25) (layer F.Cu) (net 5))
 (segment (start 142.814072 112.925928) (end 142.805204 112.934796) (width 0.25) (layer F.Cu) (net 5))
 (segment (start 151.13 109.22) (end 151.13 114.3) (width 0.25) (layer F.Cu) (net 5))
 (segment (start 153.67 106.68) (end 151.13 109.22) (width 0.25) (layer F.Cu) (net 5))
 (segment (start 151.13 109.615) (end 147.32 113.425) (width 0.25) (layer F.Cu) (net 5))
 (segment (start 151.13 109.22) (end 151.13 109.615) (width 0.25) (layer F.Cu) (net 5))
 (segment (start 146.125 109.615) (end 142.24 113.5) (width 0.25) (layer F.Cu) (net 5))
 (segment (start 151.13 109.615) (end 146.125 109.615) (width 0.25) (layer F.Cu) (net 5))
 (segment (start 141.38999 116.01086) (end 141.38999 114.35001) (width 0.25) (layer F.Cu) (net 5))
 (segment (start 146.834129 121.454999) (end 141.38999 116.01086) (width 0.25) (layer F.Cu) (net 5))
 (segment (start 141.674796 114.065204) (end 142.24 113.5) (width 0.25) (layer F.Cu) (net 5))
 (segment (start 141.38999 114.35001) (end 141.674796 114.065204) (width 0.25) (layer F.Cu) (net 5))
 (segment (start 147.794999 121.454999) (end 146.834129 121.454999) (width 0.25) (layer F.Cu) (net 5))
 (segment (start 151.629072 114.799072) (end 151.13 114.3) (width 0.25) (layer F.Cu) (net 5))
 (segment (start 154.15001 117.32001) (end 151.629072 114.799072) (width 0.25) (layer F.Cu) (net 5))
 (segment (start 154.15001 118.62318) (end 154.15001 117.32001) (width 0.25) (layer F.Cu) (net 5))
 (segment (start 152.52 120.25319) (end 154.15001 118.62318) (width 0.25) (layer F.Cu) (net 5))
 (segment (start 152.52 121.879998) (end 152.52 120.25319) (width 0.25) (layer F.Cu) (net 5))
 (segment (start 152.444999 121.954999) (end 152.52 121.879998) (width 0.25) (layer F.Cu) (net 5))
 (segment (start 151.794999 121.954999) (end 152.444999 121.954999) (width 0.25) (layer F.Cu) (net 5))
 (segment (start 139.37 123.19) (end 137.16 123.19) (width 0.25) (layer F.Cu) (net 3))
 (segment (start 122.5 123.19) (end 138.2 123.19) (width 2.9) (layer F.Cu) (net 3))
 (segment (start 160.82 123.19) (end 162.56 123.19) (width 0.25) (layer F.Cu) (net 2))
 (segment (start 162 123.19) (end 170.75 123.19) (width 2.9) (layer F.Cu) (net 2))
 (segment (start 146.85 118.11) (end 147.6 118.11) (width 0.25) (layer F.Cu) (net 6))
 (segment (start 147.32 117.64) (end 146.85 118.11) (width 0.25) (layer F.Cu) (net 6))
 (segment (start 147.32 115.175) (end 147.32 117.64) (width 0.25) (layer F.Cu) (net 6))
 (segment (start 149.069998 120.18) (end 149.044999 120.204999) (width 0.25) (layer F.Cu) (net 6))
 (segment (start 149.069998 119.579998) (end 149.069998 120.18) (width 0.25) (layer F.Cu) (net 6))
 (segment (start 147.6 118.11) (end 149.069998 119.579998) (width 0.25) (layer F.Cu) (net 6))
 (segment (start 151.13 117.64) (end 151.6 118.11) (width 0.25) (layer F.Cu) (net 4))
 (segment (start 151.13 116.05) (end 151.13 117.64) (width 0.25) (layer F.Cu) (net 4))
 (segment (start 150.544999 119.165001) (end 150.544999 120.204999) (width 0.25) (layer F.Cu) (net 4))
 (segment (start 151.6 118.11) (end 150.544999 119.165001) (width 0.25) (layer F.Cu) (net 4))
 (segment (start 159.22 123.19) (end 157.48 123.19) (width 0.25) (layer F.Cu) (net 7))
 (segment (start 154 122.954999) (end 158.2 122.954999) (width 2.9) (layer F.Cu) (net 7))
 (segment (start 151.794999 122.954999) (end 152.6 122.954999) (width 0.25) (layer F.Cu) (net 7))
 (segment (start 152.799999 122.954999) (end 153.434999 122.954999) (width 0.25) (layer F.Cu) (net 7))
 (segment (start 140.97 123.19) (end 142.24 123.19) (width 0.25) (layer F.Cu) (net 8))
 (segment (start 147.794999 122.954999) (end 147.1 122.954999) (width 0.25) (layer F.Cu) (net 8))
 (segment (start 142.175 123.19) (end 145.7 123.19) (width 2.9) (layer F.Cu) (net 8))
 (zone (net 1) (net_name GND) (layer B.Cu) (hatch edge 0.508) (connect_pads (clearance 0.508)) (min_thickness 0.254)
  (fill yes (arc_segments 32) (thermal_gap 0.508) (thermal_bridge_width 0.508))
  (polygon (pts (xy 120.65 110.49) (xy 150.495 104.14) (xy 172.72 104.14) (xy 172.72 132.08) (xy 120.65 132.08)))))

